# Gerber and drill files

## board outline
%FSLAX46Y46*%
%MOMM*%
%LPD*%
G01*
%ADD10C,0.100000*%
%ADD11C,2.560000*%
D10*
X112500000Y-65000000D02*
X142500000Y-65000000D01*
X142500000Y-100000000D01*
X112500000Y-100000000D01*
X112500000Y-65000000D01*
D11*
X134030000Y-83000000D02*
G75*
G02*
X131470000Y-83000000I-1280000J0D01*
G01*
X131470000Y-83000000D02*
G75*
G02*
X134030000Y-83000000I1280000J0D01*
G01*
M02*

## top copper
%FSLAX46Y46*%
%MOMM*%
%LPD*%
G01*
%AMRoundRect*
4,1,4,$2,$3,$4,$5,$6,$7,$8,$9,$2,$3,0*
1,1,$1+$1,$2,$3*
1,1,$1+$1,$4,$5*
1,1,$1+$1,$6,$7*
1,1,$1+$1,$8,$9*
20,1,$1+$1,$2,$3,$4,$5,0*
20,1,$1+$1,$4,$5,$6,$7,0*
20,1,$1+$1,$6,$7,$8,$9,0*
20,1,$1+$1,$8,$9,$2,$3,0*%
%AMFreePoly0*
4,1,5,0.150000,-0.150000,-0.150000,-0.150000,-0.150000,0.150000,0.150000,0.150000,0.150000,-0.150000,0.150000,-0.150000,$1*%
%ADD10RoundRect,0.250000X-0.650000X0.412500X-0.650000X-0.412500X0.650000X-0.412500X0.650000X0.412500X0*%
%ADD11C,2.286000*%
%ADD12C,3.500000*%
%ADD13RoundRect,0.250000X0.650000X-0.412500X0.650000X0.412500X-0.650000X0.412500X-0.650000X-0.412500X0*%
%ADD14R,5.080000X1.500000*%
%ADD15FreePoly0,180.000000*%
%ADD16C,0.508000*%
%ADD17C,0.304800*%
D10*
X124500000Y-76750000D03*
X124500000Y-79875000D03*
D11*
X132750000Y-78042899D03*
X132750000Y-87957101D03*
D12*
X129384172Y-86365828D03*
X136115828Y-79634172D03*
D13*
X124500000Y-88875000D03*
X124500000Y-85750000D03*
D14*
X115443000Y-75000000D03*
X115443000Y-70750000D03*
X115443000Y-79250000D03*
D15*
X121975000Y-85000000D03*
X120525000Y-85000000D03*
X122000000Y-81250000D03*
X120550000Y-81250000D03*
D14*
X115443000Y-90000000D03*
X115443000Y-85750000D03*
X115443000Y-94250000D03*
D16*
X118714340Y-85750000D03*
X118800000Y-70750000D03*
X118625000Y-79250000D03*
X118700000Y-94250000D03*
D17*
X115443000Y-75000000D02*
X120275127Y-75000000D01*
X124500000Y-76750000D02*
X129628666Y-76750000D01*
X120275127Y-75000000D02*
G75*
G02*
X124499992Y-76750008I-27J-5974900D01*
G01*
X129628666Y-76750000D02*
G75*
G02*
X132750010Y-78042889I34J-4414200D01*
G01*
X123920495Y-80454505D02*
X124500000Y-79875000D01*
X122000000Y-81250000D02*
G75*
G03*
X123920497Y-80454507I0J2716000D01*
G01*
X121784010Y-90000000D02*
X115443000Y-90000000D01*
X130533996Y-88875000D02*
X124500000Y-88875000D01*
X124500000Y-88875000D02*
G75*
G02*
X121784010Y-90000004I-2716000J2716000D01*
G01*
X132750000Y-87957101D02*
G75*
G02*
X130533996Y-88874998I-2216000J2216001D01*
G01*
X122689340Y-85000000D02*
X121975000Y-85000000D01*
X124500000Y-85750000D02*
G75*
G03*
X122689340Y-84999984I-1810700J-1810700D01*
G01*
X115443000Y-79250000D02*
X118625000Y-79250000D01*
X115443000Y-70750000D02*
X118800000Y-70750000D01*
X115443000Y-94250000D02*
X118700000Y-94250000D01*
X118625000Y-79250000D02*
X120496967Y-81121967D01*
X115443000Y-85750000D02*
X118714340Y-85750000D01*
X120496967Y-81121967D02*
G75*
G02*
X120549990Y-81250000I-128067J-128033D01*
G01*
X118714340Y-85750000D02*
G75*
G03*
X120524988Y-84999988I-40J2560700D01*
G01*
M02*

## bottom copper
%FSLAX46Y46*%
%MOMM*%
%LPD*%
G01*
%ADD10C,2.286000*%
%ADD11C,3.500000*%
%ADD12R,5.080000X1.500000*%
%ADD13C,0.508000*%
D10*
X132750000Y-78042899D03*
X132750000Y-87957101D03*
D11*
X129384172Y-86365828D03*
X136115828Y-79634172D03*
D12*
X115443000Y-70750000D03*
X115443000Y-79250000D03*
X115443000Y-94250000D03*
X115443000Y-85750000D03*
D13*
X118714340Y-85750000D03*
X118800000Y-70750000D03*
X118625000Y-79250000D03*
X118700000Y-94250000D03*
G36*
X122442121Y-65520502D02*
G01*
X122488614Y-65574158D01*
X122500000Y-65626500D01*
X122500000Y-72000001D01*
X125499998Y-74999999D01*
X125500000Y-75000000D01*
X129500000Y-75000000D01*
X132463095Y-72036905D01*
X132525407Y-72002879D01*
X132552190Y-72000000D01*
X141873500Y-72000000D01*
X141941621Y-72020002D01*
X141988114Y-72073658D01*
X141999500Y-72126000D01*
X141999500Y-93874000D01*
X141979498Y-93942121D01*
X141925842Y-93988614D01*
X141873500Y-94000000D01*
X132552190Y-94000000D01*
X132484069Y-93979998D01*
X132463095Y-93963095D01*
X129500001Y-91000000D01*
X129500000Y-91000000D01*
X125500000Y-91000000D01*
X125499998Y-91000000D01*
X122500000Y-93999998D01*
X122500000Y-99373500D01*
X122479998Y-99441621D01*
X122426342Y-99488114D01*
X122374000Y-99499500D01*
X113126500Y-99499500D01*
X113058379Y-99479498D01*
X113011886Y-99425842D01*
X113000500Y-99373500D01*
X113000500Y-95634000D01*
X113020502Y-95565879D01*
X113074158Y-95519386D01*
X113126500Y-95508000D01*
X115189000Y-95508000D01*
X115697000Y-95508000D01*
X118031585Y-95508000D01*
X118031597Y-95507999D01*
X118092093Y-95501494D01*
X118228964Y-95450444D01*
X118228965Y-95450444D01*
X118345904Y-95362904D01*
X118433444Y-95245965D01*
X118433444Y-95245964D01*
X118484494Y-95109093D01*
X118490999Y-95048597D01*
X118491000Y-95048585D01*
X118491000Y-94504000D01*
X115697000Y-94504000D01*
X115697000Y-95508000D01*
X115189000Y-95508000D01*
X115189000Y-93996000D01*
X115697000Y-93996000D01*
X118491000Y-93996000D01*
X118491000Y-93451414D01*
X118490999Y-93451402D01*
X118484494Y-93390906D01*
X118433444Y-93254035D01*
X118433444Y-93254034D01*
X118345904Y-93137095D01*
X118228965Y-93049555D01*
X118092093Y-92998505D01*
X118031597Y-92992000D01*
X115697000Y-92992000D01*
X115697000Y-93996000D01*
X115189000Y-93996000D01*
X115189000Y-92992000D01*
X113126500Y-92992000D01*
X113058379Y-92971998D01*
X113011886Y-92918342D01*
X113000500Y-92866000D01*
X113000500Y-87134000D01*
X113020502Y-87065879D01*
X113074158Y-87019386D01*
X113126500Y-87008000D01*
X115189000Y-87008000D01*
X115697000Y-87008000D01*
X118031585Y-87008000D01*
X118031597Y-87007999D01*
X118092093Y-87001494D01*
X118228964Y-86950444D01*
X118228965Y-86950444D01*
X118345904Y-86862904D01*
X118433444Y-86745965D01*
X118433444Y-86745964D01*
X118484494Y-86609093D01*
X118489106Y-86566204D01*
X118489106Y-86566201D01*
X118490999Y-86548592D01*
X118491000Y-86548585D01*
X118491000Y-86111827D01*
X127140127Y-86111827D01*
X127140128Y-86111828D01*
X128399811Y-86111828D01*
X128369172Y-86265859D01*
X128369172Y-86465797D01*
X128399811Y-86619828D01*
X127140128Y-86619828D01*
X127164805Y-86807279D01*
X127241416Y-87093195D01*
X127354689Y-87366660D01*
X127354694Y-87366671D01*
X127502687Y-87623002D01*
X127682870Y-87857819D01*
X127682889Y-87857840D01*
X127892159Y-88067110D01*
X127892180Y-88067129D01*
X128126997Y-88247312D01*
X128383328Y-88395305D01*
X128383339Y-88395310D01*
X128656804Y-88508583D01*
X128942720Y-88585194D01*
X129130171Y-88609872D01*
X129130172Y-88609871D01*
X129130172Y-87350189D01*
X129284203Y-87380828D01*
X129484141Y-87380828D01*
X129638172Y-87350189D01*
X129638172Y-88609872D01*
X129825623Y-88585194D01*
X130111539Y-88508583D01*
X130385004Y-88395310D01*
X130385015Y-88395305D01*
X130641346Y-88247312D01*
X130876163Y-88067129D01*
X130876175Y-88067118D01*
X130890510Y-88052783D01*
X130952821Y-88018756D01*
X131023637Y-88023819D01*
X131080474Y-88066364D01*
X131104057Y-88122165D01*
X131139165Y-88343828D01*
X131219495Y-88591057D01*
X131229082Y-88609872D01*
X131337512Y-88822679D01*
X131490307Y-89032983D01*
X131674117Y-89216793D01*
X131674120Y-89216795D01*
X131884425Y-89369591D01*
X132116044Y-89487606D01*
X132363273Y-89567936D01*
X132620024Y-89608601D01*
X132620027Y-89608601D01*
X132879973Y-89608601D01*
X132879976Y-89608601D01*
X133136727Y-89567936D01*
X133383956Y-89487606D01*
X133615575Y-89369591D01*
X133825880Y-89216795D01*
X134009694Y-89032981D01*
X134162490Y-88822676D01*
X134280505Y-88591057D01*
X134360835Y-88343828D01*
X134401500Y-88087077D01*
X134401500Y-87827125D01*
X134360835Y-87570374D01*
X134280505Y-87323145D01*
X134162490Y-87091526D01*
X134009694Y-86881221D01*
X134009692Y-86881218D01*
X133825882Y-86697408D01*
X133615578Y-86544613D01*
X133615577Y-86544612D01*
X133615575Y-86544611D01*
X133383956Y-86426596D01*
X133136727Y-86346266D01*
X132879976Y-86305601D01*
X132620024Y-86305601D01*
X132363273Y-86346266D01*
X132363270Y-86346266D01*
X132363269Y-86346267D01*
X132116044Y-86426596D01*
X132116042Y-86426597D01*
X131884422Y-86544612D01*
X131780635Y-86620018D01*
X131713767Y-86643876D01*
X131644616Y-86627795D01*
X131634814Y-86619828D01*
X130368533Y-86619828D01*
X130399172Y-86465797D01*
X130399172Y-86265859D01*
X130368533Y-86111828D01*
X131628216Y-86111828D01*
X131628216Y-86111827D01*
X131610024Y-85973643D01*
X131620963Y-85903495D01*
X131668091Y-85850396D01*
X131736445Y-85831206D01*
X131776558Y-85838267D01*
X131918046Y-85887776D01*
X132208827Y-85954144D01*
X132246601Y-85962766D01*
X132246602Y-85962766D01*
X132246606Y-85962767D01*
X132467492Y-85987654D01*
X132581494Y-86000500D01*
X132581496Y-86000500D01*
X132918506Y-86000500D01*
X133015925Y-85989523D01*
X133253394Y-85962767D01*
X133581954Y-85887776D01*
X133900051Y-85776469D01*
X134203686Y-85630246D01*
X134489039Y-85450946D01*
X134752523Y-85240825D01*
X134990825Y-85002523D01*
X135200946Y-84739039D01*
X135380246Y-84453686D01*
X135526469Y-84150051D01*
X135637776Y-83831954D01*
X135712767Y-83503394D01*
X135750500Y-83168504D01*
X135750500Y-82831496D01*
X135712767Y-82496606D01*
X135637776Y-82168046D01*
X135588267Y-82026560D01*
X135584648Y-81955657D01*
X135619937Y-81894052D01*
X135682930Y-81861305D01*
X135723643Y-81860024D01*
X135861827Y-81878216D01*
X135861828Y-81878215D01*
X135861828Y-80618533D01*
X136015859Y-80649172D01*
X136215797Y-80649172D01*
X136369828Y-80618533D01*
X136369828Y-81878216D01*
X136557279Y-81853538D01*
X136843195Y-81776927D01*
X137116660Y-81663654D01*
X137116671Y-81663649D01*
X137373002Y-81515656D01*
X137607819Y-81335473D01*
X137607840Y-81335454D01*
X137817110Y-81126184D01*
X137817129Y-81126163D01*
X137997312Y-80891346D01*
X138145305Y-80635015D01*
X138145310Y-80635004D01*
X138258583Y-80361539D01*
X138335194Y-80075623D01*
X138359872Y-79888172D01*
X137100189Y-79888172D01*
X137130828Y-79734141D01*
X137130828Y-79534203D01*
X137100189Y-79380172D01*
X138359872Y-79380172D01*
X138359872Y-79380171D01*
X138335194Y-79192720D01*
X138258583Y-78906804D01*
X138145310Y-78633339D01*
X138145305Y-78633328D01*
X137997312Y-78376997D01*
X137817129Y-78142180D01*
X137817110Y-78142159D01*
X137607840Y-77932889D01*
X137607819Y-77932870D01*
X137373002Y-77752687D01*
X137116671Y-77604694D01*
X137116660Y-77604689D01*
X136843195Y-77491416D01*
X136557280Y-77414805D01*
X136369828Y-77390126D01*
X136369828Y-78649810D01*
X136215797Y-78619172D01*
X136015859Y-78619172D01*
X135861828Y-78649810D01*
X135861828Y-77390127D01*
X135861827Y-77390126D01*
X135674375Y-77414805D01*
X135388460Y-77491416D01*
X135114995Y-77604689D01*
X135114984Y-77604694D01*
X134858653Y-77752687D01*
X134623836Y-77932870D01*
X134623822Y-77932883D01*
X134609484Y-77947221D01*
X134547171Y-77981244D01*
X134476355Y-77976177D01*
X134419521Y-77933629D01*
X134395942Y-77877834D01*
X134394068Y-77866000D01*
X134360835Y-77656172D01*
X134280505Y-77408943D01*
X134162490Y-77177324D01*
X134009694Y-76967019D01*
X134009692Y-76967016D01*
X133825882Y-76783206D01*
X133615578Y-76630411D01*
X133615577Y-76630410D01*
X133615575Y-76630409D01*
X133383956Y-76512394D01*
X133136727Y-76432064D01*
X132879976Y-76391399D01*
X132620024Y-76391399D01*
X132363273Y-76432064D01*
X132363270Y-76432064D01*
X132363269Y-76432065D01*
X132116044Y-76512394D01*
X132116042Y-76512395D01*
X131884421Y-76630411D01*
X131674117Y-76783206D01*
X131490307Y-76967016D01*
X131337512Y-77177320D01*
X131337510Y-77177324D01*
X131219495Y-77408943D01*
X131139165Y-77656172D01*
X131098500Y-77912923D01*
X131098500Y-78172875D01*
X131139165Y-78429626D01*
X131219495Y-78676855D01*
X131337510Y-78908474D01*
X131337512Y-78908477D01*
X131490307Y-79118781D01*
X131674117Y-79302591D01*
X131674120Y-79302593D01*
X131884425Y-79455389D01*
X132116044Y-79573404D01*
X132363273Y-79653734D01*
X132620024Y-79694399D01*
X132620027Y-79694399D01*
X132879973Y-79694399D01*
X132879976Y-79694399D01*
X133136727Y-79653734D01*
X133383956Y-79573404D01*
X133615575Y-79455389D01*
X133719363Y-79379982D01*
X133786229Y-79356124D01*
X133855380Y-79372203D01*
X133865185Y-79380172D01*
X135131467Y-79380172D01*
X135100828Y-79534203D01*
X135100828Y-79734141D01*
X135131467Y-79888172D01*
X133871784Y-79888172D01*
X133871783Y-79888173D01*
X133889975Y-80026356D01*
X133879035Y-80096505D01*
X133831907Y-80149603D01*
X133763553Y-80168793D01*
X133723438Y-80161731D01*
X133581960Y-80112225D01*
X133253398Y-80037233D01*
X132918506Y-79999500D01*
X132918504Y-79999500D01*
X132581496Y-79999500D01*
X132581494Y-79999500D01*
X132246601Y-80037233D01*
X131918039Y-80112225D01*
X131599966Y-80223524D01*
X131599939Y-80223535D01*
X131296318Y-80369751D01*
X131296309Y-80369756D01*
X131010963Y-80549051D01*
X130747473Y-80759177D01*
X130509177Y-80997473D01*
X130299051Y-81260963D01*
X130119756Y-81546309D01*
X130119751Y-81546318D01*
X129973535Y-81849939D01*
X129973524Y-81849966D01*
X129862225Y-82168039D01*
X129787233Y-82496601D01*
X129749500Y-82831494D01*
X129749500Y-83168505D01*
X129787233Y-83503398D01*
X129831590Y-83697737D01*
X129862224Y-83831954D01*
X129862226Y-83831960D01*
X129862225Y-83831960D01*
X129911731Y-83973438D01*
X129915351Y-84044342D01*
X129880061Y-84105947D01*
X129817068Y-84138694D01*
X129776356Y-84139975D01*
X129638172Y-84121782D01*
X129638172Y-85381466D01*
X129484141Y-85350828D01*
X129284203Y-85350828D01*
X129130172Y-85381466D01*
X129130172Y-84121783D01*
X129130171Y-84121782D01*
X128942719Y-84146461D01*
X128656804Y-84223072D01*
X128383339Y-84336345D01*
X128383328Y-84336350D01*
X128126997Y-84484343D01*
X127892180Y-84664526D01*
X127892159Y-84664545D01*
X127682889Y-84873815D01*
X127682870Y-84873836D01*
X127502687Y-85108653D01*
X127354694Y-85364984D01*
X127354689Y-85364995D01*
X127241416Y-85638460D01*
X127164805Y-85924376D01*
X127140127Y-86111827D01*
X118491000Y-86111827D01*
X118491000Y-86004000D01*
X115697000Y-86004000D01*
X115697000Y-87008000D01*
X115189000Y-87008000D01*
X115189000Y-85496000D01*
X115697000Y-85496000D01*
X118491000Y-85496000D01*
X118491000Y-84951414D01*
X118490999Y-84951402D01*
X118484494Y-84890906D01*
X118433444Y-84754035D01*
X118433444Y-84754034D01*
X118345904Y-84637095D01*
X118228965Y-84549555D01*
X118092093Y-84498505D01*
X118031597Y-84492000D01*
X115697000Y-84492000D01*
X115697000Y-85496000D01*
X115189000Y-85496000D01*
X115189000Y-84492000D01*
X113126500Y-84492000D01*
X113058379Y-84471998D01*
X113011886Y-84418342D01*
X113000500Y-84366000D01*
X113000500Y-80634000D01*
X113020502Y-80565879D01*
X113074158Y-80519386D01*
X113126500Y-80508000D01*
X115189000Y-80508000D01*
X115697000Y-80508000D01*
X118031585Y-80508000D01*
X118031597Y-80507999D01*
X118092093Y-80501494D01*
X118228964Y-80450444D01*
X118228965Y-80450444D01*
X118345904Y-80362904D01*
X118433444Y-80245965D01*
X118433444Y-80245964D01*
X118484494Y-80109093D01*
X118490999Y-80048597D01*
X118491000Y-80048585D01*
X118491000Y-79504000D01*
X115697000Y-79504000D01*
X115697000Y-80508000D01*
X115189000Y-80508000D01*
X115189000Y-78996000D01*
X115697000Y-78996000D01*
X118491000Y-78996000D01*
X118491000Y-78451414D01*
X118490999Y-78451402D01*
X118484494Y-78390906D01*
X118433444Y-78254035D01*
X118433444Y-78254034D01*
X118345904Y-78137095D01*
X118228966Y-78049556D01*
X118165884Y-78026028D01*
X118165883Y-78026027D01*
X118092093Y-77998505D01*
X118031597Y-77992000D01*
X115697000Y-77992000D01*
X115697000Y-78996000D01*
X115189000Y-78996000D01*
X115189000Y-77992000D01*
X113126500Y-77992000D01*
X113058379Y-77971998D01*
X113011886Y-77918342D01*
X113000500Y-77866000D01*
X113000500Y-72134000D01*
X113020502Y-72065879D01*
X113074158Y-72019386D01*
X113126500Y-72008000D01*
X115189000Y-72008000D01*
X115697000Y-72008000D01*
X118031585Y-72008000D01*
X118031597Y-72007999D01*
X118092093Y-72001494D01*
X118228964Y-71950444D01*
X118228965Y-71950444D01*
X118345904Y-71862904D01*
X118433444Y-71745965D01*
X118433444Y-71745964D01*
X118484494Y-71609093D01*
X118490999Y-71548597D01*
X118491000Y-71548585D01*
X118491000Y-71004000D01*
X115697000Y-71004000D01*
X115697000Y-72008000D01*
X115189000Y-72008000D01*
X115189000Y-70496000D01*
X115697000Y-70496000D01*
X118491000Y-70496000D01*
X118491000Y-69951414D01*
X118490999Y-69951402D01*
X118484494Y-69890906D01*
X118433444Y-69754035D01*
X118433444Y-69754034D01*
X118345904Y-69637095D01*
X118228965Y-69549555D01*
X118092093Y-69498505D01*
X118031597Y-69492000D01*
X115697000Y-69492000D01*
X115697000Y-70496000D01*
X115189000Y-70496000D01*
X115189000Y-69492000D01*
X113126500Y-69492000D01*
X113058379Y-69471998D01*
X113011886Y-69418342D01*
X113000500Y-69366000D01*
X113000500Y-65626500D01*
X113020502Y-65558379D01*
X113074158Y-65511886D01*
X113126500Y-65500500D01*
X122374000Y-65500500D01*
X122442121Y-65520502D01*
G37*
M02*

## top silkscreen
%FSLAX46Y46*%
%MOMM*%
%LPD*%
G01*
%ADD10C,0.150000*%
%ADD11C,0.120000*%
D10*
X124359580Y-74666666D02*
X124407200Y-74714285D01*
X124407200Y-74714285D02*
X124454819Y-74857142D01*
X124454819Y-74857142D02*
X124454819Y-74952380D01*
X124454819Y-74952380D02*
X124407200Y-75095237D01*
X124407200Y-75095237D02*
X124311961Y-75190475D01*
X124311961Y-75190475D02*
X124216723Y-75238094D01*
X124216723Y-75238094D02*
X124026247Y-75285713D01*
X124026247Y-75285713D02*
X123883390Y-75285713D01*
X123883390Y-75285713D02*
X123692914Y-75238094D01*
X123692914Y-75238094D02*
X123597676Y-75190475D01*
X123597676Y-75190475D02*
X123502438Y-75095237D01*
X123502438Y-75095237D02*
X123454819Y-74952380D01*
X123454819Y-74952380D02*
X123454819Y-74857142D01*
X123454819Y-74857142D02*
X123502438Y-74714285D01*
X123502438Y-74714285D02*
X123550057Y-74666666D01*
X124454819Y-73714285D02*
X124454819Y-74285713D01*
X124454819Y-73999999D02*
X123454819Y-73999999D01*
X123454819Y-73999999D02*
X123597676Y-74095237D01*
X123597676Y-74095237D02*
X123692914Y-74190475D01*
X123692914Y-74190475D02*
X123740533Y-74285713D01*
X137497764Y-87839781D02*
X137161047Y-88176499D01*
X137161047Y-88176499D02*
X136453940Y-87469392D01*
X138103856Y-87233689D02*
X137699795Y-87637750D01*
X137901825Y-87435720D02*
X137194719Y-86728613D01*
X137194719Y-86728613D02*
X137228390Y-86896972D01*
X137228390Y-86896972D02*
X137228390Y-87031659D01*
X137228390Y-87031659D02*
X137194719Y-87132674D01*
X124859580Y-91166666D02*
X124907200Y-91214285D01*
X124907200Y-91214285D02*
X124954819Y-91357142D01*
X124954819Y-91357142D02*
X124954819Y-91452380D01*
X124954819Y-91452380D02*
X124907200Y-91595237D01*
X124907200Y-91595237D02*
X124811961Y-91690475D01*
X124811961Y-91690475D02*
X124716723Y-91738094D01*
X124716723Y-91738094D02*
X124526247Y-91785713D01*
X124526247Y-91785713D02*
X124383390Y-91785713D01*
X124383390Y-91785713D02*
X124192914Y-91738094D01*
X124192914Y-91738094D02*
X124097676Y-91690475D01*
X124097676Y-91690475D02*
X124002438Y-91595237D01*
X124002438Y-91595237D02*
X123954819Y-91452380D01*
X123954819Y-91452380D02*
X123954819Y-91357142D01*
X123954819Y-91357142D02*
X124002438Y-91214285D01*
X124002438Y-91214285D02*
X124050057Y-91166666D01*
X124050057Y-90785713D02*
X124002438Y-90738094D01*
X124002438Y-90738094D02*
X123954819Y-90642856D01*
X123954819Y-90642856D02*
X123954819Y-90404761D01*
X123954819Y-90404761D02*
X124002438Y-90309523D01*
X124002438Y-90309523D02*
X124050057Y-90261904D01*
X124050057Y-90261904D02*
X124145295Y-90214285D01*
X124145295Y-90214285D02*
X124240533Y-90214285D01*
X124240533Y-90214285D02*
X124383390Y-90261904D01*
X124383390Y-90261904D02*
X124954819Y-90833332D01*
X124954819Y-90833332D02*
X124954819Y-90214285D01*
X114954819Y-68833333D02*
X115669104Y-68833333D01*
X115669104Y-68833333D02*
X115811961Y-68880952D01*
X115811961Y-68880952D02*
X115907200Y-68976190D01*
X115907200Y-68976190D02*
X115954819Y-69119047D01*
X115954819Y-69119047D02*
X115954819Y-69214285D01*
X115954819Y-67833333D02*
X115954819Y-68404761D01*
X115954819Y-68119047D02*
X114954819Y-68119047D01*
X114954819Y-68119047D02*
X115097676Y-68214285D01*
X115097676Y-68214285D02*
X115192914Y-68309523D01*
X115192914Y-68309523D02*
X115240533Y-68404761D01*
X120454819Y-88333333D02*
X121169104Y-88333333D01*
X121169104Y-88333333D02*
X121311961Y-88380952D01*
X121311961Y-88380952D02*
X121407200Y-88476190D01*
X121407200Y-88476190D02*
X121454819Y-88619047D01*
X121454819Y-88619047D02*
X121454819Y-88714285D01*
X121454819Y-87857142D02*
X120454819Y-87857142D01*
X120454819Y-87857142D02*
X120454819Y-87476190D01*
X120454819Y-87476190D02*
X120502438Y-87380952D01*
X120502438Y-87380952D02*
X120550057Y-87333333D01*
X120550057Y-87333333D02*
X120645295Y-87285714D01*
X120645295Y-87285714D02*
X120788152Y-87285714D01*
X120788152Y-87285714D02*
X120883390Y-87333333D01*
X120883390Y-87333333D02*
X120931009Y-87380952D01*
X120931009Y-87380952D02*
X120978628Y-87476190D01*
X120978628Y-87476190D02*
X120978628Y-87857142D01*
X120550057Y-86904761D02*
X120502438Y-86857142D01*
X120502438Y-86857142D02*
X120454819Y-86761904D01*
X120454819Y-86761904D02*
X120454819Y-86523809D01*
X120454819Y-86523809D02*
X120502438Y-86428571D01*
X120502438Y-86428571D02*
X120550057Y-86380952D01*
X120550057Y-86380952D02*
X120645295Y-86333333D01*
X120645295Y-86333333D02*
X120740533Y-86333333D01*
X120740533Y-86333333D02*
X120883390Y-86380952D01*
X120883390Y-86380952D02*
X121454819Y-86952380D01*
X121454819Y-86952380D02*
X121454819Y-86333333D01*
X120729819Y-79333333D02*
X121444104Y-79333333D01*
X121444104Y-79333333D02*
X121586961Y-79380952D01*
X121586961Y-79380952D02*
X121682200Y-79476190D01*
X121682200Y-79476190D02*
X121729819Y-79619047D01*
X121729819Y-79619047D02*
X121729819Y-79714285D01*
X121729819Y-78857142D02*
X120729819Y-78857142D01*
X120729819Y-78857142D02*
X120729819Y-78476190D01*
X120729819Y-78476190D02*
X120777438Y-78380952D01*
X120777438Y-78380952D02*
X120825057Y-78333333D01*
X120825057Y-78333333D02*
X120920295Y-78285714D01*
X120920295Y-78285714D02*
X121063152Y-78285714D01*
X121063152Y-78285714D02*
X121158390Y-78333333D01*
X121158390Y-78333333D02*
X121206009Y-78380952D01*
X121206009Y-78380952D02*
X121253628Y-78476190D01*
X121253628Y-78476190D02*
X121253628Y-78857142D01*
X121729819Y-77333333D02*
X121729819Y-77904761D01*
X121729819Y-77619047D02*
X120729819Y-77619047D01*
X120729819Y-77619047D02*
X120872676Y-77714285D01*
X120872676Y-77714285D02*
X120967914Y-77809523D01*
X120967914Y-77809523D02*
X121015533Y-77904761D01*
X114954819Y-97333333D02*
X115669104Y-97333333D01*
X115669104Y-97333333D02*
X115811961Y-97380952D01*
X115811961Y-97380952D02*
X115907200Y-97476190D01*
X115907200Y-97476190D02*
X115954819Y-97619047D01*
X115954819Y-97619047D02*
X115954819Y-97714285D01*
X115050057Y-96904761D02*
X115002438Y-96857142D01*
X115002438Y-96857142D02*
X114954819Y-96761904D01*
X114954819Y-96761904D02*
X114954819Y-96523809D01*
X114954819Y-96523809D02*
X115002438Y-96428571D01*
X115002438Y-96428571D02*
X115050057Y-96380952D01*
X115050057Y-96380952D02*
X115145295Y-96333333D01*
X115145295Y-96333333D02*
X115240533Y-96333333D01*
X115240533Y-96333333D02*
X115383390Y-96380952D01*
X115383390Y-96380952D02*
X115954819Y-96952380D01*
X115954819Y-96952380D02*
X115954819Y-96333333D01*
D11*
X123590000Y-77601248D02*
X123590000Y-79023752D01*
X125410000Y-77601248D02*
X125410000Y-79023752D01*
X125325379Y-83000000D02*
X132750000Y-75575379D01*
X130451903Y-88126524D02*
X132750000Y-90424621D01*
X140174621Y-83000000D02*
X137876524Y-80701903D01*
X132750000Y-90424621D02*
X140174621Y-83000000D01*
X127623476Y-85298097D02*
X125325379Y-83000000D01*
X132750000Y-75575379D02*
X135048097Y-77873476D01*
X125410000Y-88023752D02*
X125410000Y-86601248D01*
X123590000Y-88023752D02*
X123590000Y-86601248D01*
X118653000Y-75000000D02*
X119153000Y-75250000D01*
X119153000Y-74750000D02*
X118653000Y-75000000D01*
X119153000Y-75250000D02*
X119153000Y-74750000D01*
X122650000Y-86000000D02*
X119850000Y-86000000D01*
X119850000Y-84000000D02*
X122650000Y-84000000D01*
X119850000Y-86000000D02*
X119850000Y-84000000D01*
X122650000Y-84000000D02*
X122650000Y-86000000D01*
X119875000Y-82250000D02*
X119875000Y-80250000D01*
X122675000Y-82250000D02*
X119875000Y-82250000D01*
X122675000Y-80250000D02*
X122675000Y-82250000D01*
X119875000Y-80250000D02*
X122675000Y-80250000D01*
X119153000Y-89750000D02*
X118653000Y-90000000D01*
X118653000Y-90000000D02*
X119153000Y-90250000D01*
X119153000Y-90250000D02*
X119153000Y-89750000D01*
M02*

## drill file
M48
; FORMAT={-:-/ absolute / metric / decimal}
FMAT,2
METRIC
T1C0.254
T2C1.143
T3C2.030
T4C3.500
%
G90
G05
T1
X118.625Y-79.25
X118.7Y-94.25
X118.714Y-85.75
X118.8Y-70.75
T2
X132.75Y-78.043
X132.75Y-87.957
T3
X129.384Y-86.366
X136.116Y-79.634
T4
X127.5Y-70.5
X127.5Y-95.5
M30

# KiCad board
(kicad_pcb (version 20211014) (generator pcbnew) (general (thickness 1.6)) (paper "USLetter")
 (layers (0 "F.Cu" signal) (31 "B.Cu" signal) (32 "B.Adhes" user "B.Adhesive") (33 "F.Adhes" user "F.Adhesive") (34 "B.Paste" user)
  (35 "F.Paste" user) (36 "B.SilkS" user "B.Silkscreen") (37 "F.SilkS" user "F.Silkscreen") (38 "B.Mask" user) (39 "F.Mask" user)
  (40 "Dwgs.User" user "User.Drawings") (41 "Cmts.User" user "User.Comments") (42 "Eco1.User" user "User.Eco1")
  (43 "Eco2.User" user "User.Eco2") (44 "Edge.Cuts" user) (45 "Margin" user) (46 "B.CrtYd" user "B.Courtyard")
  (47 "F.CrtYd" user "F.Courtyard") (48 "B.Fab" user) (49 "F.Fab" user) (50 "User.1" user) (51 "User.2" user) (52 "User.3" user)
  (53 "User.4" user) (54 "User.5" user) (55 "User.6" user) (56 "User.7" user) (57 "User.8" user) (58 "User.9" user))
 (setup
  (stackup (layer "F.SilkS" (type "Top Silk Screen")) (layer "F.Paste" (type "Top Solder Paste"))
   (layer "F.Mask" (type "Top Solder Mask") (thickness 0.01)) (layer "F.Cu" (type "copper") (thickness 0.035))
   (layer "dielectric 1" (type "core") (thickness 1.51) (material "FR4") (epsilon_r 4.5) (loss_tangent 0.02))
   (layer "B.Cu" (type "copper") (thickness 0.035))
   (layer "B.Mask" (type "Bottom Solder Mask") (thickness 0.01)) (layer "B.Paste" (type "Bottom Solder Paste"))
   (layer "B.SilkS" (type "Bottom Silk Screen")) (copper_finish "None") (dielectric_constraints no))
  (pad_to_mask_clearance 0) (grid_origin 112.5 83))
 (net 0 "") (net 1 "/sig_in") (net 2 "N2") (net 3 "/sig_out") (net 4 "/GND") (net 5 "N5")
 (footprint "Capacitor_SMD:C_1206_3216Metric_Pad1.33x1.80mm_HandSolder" (layer "F.Cu") (at 124.5 78.3125 -90)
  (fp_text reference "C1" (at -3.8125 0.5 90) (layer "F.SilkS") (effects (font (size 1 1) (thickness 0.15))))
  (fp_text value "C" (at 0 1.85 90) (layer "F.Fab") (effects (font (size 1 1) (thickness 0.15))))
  (fp_line (start -0.711252 0.91) (end 0.711252 0.91) (layer "F.SilkS") (width 0.12))
  (fp_line (start -0.711252 -0.91) (end 0.711252 -0.91) (layer "F.SilkS") (width 0.12))
  (pad "1" smd roundrect (at -1.5625 0 270) (size 1.325 1.8) (layers "F.Cu" "F.Paste" "F.Mask") (roundrect_rratio 0.1886792453)
   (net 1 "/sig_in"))
  (pad "2" smd roundrect (at 1.5625 0 270) (size 1.325 1.8) (layers "F.Cu" "F.Paste" "F.Mask") (roundrect_rratio 0.1886792453) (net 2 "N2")))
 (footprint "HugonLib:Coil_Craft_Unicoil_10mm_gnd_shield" (layer "F.Cu") (at 132.75 83 45)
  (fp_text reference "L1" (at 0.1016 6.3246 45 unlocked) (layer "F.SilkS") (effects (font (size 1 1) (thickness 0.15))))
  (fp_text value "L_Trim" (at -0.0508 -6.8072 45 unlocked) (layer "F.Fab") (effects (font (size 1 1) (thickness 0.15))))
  (fp_line (start -5.25 -5.25) (end 5.25 -5.25) (layer "F.SilkS") (width 0.12))
  (fp_line (start -5.25 2) (end -5.25 5.25) (layer "F.SilkS") (width 0.12))
  (fp_line (start 5.25 5.25) (end 5.25 2) (layer "F.SilkS") (width 0.12))
  (fp_line (start -5.25 5.25) (end 5.25 5.25) (layer "F.SilkS") (width 0.12))
  (fp_line (start -5.25 -2) (end -5.25 -5.25) (layer "F.SilkS") (width 0.12))
  (fp_line (start 5.25 -5.25) (end 5.25 -2) (layer "F.SilkS") (width 0.12))
  (fp_circle (center 0 0) (end 2.5 0) (layer "Edge.Cuts") (width 0.12) (fill solid))
  (pad "1" thru_hole circle (at 3.5052 -3.5052 45) (size 2.286 2.286) (drill 1.143) (layers *.Cu *.Mask) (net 1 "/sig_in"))
  (pad "2" thru_hole circle (at -3.5052 3.5052 45) (size 2.286 2.286) (drill 1.143) (layers *.Cu *.Mask) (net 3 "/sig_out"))
  (pad "GND" thru_hole circle (at -4.76 0 45) (size 3.5 3.5) (drill 2.03) (layers *.Cu *.Mask) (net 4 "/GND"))
  (pad "GND" thru_hole circle (at 4.76 0 45) (size 3.5 3.5) (drill 2.03) (layers *.Cu *.Mask) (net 4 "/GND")))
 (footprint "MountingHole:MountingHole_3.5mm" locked (layer "F.Cu") (at 127.5 70.5)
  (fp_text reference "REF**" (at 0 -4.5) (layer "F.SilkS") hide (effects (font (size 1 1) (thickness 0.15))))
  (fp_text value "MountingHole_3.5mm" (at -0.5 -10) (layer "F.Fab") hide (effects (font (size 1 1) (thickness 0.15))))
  (pad "" np_thru_hole circle locked (at 0 0) (size 3.5 3.5) (drill 3.5) (layers *.Cu *.Mask)))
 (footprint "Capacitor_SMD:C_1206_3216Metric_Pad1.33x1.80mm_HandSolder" (layer "F.Cu") (at 124.5 87.3125 90)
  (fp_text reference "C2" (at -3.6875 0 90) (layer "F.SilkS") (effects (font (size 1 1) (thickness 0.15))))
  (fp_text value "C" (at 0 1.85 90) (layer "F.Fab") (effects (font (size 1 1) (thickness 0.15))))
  (fp_line (start -0.711252 0.91) (end 0.711252 0.91) (layer "F.SilkS") (width 0.12))
  (fp_line (start -0.711252 -0.91) (end 0.711252 -0.91) (layer "F.SilkS") (width 0.12))
  (pad "1" smd roundrect (at -1.5625 0 90) (size 1.325 1.8) (layers "F.Cu" "F.Paste" "F.Mask") (roundrect_rratio 0.1886792453)
   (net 3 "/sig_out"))
  (pad "2" smd roundrect (at 1.5625 0 90) (size 1.325 1.8) (layers "F.Cu" "F.Paste" "F.Mask") (roundrect_rratio 0.1886792453) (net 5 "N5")))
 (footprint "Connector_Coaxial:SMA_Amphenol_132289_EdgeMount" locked (layer "F.Cu") (at 115.443 75 180)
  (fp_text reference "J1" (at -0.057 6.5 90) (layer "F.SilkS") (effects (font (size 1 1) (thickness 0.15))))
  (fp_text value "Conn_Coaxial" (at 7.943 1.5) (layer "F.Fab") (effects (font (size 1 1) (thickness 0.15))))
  (fp_line (start -3.21 0) (end -3.71 -0.25) (layer "F.SilkS") (width 0.12))
  (fp_line (start -3.71 0.25) (end -3.21 0) (layer "F.SilkS") (width 0.12))
  (fp_line (start -3.71 -0.25) (end -3.71 0.25) (layer "F.SilkS") (width 0.12))
  (pad "1" smd rect locked (at 0 0 270) (size 1.5 5.08) (layers "F.Cu" "F.Paste" "F.Mask") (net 1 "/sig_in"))
  (pad "2" smd rect locked (at 0 4.25 270) (size 1.5 5.08) (layers "F.Cu" "F.Paste" "F.Mask") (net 4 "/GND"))
  (pad "2" smd rect locked (at 0 4.25 270) (size 1.5 5.08) (layers "B.Cu" "B.Paste" "B.Mask") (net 4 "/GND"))
  (pad "2" smd rect locked (at 0 -4.25 270) (size 1.5 5.08) (layers "B.Cu" "B.Paste" "B.Mask") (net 4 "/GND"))
  (pad "2" smd rect locked (at 0 -4.25 270) (size 1.5 5.08) (layers "F.Cu" "F.Paste" "F.Mask") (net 4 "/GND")))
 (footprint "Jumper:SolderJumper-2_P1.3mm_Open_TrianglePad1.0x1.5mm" (layer "F.Cu") (at 121.25 85 180)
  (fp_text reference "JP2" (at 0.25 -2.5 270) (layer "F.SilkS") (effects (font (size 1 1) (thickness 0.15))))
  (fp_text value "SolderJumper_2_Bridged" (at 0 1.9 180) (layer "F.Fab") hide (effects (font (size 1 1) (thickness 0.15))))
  (fp_line (start -1.4 -1) (end 1.4 -1) (layer "F.SilkS") (width 0.12))
  (fp_line (start 1.4 1) (end -1.4 1) (layer "F.SilkS") (width 0.12))
  (fp_line (start 1.4 -1) (end 1.4 1) (layer "F.SilkS") (width 0.12))
  (fp_line (start -1.4 1) (end -1.4 -1) (layer "F.SilkS") (width 0.12))
  (pad "1" smd custom (at -0.725 0 180) (size 0.3 0.3) (layers "F.Cu" "F.Mask") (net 5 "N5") (zone_connect 2)
   (options (clearance outline) (anchor rect)) (primitives))
  (pad "2" smd custom (at 0.725 0 180) (size 0.3 0.3) (layers "F.Cu" "F.Mask") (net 4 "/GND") (zone_connect 2)
   (options (clearance outline) (anchor rect)) (primitives)))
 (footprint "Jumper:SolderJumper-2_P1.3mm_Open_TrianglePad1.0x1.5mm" (layer "F.Cu") (at 121.275 81.25 180)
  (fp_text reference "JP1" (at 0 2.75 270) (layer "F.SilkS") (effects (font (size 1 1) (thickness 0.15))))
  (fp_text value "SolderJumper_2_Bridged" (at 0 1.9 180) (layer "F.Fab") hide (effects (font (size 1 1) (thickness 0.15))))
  (fp_line (start 1.4 -1) (end 1.4 1) (layer "F.SilkS") (width 0.12))
  (fp_line (start -1.4 -1) (end 1.4 -1) (layer "F.SilkS") (width 0.12))
  (fp_line (start -1.4 1) (end -1.4 -1) (layer "F.SilkS") (width 0.12))
  (fp_line (start 1.4 1) (end -1.4 1) (layer "F.SilkS") (width 0.12))
  (pad "1" smd custom (at -0.725 0 180) (size 0.3 0.3) (layers "F.Cu" "F.Mask") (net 2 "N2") (zone_connect 2)
   (options (clearance outline) (anchor rect)) (primitives))
  (pad "2" smd custom (at 0.725 0 180) (size 0.3 0.3) (layers "F.Cu" "F.Mask") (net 4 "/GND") (zone_connect 2)
   (options (clearance outline) (anchor rect)) (primitives)))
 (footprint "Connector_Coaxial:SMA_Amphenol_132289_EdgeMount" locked (layer "F.Cu") (at 115.443 90 180)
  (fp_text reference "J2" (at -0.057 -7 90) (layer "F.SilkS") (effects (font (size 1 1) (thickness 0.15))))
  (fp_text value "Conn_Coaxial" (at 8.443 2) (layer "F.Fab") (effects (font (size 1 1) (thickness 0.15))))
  (fp_line (start -3.71 0.25) (end -3.21 0) (layer "F.SilkS") (width 0.12))
  (fp_line (start -3.21 0) (end -3.71 -0.25) (layer "F.SilkS") (width 0.12))
  (fp_line (start -3.71 -0.25) (end -3.71 0.25) (layer "F.SilkS") (width 0.12))
  (pad "1" smd rect locked (at 0 0 270) (size 1.5 5.08) (layers "F.Cu" "F.Paste" "F.Mask") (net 3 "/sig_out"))
  (pad "2" smd rect locked (at 0 -4.25 270) (size 1.5 5.08) (layers "B.Cu" "B.Paste" "B.Mask") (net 4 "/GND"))
  (pad "2" smd rect locked (at 0 4.25 270) (size 1.5 5.08) (layers "B.Cu" "B.Paste" "B.Mask") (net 4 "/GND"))
  (pad "2" smd rect locked (at 0 4.25 270) (size 1.5 5.08) (layers "F.Cu" "F.Paste" "F.Mask") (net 4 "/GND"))
  (pad "2" smd rect locked (at 0 -4.25 270) (size 1.5 5.08) (layers "F.Cu" "F.Paste" "F.Mask") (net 4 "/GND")))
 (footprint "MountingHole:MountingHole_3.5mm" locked (layer "F.Cu") (at 127.5 95.5)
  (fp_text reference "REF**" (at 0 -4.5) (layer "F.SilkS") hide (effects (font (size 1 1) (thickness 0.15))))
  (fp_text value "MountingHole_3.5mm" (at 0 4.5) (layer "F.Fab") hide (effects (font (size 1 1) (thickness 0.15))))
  (pad "" np_thru_hole circle locked (at 0 0) (size 3.5 3.5) (drill 3.5) (layers *.Cu *.Mask)))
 (gr_rect locked (start 112.5 65) (end 142.5 100) (layer "Edge.Cuts") (width 0.1) (fill none))
 (segment (start 115.443 75) (end 120.275127 75) (width 0.3048) (layer "F.Cu") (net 1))
 (segment (start 124.5 76.75) (end 129.628666 76.75) (width 0.3048) (layer "F.Cu") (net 1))
 (arc (start 120.275127 75) (mid 122.561611 75.45481) (end 124.5 76.75) (width 0.3048) (layer "F.Cu") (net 1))
 (arc (start 129.628666 76.75) (mid 131.317919 77.086014) (end 132.75 78.042899) (width 0.3048) (layer "F.Cu") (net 1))
 (segment (start 123.920495 80.454505) (end 124.5 79.875) (width 0.3048) (layer "F.Cu") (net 2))
 (arc (start 122 81.25) (mid 123.039364 81.043258) (end 123.920495 80.454505) (width 0.3048) (layer "F.Cu") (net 2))
 (segment (start 121.78401 90) (end 115.443 90) (width 0.3048) (layer "F.Cu") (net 3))
 (segment (start 130.533996 88.875) (end 124.5 88.875) (width 0.3048) (layer "F.Cu") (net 3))
 (arc (start 124.5 88.875) (mid 123.253893 89.707622) (end 121.78401 90) (width 0.3048) (layer "F.Cu") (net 3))
 (arc (start 132.75 87.957101) (mid 131.733289 88.636446) (end 130.533996 88.875) (width 0.3048) (layer "F.Cu") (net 3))
 (segment (start 122.68934 85) (end 121.975 85) (width 0.3048) (layer "F.Cu") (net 5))
 (arc (start 124.5 85.75) (mid 123.669262 85.194918) (end 122.68934 85) (width 0.3048) (layer "F.Cu") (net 5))
 (segment (start 115.443 79.25) (end 118.625 79.25) (width 0.3048) (layer "F.Cu") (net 4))
 (segment (start 115.443 70.75) (end 118.8 70.75) (width 0.3048) (layer "F.Cu") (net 4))
 (segment (start 115.443 94.25) (end 118.7 94.25) (width 0.3048) (layer "F.Cu") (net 4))
 (segment (start 118.625 79.25) (end 120.496967 81.121967) (width 0.3048) (layer "F.Cu") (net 4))
 (segment (start 115.443 85.75) (end 118.71434 85.75) (width 0.3048) (layer "F.Cu") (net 4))
 (via (at 118.71434 85.75) (size 0.508) (drill 0.254) (layers "F.Cu" "B.Cu") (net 4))
 (via (at 118.8 70.75) (size 0.508) (drill 0.254) (layers "F.Cu" "B.Cu") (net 4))
 (via (at 118.625 79.25) (size 0.508) (drill 0.254) (layers "F.Cu" "B.Cu") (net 4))
 (via (at 118.7 94.25) (size 0.508) (drill 0.254) (layers "F.Cu" "B.Cu") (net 4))
 (arc (start 120.496967 81.121967) (mid 120.536217 81.180709) (end 120.55 81.25) (width 0.3048) (layer "F.Cu") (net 4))
 (arc (start 118.71434 85.75) (mid 119.694262 85.555081) (end 120.525 85) (width 0.3048) (layer "F.Cu") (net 4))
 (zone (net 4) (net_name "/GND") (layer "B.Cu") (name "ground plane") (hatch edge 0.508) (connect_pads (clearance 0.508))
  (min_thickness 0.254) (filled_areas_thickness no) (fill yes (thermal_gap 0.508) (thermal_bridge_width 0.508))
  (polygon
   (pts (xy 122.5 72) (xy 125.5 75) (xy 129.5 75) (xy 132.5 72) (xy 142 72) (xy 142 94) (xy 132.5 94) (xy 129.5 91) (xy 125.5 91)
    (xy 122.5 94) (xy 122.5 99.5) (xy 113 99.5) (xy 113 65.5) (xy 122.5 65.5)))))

